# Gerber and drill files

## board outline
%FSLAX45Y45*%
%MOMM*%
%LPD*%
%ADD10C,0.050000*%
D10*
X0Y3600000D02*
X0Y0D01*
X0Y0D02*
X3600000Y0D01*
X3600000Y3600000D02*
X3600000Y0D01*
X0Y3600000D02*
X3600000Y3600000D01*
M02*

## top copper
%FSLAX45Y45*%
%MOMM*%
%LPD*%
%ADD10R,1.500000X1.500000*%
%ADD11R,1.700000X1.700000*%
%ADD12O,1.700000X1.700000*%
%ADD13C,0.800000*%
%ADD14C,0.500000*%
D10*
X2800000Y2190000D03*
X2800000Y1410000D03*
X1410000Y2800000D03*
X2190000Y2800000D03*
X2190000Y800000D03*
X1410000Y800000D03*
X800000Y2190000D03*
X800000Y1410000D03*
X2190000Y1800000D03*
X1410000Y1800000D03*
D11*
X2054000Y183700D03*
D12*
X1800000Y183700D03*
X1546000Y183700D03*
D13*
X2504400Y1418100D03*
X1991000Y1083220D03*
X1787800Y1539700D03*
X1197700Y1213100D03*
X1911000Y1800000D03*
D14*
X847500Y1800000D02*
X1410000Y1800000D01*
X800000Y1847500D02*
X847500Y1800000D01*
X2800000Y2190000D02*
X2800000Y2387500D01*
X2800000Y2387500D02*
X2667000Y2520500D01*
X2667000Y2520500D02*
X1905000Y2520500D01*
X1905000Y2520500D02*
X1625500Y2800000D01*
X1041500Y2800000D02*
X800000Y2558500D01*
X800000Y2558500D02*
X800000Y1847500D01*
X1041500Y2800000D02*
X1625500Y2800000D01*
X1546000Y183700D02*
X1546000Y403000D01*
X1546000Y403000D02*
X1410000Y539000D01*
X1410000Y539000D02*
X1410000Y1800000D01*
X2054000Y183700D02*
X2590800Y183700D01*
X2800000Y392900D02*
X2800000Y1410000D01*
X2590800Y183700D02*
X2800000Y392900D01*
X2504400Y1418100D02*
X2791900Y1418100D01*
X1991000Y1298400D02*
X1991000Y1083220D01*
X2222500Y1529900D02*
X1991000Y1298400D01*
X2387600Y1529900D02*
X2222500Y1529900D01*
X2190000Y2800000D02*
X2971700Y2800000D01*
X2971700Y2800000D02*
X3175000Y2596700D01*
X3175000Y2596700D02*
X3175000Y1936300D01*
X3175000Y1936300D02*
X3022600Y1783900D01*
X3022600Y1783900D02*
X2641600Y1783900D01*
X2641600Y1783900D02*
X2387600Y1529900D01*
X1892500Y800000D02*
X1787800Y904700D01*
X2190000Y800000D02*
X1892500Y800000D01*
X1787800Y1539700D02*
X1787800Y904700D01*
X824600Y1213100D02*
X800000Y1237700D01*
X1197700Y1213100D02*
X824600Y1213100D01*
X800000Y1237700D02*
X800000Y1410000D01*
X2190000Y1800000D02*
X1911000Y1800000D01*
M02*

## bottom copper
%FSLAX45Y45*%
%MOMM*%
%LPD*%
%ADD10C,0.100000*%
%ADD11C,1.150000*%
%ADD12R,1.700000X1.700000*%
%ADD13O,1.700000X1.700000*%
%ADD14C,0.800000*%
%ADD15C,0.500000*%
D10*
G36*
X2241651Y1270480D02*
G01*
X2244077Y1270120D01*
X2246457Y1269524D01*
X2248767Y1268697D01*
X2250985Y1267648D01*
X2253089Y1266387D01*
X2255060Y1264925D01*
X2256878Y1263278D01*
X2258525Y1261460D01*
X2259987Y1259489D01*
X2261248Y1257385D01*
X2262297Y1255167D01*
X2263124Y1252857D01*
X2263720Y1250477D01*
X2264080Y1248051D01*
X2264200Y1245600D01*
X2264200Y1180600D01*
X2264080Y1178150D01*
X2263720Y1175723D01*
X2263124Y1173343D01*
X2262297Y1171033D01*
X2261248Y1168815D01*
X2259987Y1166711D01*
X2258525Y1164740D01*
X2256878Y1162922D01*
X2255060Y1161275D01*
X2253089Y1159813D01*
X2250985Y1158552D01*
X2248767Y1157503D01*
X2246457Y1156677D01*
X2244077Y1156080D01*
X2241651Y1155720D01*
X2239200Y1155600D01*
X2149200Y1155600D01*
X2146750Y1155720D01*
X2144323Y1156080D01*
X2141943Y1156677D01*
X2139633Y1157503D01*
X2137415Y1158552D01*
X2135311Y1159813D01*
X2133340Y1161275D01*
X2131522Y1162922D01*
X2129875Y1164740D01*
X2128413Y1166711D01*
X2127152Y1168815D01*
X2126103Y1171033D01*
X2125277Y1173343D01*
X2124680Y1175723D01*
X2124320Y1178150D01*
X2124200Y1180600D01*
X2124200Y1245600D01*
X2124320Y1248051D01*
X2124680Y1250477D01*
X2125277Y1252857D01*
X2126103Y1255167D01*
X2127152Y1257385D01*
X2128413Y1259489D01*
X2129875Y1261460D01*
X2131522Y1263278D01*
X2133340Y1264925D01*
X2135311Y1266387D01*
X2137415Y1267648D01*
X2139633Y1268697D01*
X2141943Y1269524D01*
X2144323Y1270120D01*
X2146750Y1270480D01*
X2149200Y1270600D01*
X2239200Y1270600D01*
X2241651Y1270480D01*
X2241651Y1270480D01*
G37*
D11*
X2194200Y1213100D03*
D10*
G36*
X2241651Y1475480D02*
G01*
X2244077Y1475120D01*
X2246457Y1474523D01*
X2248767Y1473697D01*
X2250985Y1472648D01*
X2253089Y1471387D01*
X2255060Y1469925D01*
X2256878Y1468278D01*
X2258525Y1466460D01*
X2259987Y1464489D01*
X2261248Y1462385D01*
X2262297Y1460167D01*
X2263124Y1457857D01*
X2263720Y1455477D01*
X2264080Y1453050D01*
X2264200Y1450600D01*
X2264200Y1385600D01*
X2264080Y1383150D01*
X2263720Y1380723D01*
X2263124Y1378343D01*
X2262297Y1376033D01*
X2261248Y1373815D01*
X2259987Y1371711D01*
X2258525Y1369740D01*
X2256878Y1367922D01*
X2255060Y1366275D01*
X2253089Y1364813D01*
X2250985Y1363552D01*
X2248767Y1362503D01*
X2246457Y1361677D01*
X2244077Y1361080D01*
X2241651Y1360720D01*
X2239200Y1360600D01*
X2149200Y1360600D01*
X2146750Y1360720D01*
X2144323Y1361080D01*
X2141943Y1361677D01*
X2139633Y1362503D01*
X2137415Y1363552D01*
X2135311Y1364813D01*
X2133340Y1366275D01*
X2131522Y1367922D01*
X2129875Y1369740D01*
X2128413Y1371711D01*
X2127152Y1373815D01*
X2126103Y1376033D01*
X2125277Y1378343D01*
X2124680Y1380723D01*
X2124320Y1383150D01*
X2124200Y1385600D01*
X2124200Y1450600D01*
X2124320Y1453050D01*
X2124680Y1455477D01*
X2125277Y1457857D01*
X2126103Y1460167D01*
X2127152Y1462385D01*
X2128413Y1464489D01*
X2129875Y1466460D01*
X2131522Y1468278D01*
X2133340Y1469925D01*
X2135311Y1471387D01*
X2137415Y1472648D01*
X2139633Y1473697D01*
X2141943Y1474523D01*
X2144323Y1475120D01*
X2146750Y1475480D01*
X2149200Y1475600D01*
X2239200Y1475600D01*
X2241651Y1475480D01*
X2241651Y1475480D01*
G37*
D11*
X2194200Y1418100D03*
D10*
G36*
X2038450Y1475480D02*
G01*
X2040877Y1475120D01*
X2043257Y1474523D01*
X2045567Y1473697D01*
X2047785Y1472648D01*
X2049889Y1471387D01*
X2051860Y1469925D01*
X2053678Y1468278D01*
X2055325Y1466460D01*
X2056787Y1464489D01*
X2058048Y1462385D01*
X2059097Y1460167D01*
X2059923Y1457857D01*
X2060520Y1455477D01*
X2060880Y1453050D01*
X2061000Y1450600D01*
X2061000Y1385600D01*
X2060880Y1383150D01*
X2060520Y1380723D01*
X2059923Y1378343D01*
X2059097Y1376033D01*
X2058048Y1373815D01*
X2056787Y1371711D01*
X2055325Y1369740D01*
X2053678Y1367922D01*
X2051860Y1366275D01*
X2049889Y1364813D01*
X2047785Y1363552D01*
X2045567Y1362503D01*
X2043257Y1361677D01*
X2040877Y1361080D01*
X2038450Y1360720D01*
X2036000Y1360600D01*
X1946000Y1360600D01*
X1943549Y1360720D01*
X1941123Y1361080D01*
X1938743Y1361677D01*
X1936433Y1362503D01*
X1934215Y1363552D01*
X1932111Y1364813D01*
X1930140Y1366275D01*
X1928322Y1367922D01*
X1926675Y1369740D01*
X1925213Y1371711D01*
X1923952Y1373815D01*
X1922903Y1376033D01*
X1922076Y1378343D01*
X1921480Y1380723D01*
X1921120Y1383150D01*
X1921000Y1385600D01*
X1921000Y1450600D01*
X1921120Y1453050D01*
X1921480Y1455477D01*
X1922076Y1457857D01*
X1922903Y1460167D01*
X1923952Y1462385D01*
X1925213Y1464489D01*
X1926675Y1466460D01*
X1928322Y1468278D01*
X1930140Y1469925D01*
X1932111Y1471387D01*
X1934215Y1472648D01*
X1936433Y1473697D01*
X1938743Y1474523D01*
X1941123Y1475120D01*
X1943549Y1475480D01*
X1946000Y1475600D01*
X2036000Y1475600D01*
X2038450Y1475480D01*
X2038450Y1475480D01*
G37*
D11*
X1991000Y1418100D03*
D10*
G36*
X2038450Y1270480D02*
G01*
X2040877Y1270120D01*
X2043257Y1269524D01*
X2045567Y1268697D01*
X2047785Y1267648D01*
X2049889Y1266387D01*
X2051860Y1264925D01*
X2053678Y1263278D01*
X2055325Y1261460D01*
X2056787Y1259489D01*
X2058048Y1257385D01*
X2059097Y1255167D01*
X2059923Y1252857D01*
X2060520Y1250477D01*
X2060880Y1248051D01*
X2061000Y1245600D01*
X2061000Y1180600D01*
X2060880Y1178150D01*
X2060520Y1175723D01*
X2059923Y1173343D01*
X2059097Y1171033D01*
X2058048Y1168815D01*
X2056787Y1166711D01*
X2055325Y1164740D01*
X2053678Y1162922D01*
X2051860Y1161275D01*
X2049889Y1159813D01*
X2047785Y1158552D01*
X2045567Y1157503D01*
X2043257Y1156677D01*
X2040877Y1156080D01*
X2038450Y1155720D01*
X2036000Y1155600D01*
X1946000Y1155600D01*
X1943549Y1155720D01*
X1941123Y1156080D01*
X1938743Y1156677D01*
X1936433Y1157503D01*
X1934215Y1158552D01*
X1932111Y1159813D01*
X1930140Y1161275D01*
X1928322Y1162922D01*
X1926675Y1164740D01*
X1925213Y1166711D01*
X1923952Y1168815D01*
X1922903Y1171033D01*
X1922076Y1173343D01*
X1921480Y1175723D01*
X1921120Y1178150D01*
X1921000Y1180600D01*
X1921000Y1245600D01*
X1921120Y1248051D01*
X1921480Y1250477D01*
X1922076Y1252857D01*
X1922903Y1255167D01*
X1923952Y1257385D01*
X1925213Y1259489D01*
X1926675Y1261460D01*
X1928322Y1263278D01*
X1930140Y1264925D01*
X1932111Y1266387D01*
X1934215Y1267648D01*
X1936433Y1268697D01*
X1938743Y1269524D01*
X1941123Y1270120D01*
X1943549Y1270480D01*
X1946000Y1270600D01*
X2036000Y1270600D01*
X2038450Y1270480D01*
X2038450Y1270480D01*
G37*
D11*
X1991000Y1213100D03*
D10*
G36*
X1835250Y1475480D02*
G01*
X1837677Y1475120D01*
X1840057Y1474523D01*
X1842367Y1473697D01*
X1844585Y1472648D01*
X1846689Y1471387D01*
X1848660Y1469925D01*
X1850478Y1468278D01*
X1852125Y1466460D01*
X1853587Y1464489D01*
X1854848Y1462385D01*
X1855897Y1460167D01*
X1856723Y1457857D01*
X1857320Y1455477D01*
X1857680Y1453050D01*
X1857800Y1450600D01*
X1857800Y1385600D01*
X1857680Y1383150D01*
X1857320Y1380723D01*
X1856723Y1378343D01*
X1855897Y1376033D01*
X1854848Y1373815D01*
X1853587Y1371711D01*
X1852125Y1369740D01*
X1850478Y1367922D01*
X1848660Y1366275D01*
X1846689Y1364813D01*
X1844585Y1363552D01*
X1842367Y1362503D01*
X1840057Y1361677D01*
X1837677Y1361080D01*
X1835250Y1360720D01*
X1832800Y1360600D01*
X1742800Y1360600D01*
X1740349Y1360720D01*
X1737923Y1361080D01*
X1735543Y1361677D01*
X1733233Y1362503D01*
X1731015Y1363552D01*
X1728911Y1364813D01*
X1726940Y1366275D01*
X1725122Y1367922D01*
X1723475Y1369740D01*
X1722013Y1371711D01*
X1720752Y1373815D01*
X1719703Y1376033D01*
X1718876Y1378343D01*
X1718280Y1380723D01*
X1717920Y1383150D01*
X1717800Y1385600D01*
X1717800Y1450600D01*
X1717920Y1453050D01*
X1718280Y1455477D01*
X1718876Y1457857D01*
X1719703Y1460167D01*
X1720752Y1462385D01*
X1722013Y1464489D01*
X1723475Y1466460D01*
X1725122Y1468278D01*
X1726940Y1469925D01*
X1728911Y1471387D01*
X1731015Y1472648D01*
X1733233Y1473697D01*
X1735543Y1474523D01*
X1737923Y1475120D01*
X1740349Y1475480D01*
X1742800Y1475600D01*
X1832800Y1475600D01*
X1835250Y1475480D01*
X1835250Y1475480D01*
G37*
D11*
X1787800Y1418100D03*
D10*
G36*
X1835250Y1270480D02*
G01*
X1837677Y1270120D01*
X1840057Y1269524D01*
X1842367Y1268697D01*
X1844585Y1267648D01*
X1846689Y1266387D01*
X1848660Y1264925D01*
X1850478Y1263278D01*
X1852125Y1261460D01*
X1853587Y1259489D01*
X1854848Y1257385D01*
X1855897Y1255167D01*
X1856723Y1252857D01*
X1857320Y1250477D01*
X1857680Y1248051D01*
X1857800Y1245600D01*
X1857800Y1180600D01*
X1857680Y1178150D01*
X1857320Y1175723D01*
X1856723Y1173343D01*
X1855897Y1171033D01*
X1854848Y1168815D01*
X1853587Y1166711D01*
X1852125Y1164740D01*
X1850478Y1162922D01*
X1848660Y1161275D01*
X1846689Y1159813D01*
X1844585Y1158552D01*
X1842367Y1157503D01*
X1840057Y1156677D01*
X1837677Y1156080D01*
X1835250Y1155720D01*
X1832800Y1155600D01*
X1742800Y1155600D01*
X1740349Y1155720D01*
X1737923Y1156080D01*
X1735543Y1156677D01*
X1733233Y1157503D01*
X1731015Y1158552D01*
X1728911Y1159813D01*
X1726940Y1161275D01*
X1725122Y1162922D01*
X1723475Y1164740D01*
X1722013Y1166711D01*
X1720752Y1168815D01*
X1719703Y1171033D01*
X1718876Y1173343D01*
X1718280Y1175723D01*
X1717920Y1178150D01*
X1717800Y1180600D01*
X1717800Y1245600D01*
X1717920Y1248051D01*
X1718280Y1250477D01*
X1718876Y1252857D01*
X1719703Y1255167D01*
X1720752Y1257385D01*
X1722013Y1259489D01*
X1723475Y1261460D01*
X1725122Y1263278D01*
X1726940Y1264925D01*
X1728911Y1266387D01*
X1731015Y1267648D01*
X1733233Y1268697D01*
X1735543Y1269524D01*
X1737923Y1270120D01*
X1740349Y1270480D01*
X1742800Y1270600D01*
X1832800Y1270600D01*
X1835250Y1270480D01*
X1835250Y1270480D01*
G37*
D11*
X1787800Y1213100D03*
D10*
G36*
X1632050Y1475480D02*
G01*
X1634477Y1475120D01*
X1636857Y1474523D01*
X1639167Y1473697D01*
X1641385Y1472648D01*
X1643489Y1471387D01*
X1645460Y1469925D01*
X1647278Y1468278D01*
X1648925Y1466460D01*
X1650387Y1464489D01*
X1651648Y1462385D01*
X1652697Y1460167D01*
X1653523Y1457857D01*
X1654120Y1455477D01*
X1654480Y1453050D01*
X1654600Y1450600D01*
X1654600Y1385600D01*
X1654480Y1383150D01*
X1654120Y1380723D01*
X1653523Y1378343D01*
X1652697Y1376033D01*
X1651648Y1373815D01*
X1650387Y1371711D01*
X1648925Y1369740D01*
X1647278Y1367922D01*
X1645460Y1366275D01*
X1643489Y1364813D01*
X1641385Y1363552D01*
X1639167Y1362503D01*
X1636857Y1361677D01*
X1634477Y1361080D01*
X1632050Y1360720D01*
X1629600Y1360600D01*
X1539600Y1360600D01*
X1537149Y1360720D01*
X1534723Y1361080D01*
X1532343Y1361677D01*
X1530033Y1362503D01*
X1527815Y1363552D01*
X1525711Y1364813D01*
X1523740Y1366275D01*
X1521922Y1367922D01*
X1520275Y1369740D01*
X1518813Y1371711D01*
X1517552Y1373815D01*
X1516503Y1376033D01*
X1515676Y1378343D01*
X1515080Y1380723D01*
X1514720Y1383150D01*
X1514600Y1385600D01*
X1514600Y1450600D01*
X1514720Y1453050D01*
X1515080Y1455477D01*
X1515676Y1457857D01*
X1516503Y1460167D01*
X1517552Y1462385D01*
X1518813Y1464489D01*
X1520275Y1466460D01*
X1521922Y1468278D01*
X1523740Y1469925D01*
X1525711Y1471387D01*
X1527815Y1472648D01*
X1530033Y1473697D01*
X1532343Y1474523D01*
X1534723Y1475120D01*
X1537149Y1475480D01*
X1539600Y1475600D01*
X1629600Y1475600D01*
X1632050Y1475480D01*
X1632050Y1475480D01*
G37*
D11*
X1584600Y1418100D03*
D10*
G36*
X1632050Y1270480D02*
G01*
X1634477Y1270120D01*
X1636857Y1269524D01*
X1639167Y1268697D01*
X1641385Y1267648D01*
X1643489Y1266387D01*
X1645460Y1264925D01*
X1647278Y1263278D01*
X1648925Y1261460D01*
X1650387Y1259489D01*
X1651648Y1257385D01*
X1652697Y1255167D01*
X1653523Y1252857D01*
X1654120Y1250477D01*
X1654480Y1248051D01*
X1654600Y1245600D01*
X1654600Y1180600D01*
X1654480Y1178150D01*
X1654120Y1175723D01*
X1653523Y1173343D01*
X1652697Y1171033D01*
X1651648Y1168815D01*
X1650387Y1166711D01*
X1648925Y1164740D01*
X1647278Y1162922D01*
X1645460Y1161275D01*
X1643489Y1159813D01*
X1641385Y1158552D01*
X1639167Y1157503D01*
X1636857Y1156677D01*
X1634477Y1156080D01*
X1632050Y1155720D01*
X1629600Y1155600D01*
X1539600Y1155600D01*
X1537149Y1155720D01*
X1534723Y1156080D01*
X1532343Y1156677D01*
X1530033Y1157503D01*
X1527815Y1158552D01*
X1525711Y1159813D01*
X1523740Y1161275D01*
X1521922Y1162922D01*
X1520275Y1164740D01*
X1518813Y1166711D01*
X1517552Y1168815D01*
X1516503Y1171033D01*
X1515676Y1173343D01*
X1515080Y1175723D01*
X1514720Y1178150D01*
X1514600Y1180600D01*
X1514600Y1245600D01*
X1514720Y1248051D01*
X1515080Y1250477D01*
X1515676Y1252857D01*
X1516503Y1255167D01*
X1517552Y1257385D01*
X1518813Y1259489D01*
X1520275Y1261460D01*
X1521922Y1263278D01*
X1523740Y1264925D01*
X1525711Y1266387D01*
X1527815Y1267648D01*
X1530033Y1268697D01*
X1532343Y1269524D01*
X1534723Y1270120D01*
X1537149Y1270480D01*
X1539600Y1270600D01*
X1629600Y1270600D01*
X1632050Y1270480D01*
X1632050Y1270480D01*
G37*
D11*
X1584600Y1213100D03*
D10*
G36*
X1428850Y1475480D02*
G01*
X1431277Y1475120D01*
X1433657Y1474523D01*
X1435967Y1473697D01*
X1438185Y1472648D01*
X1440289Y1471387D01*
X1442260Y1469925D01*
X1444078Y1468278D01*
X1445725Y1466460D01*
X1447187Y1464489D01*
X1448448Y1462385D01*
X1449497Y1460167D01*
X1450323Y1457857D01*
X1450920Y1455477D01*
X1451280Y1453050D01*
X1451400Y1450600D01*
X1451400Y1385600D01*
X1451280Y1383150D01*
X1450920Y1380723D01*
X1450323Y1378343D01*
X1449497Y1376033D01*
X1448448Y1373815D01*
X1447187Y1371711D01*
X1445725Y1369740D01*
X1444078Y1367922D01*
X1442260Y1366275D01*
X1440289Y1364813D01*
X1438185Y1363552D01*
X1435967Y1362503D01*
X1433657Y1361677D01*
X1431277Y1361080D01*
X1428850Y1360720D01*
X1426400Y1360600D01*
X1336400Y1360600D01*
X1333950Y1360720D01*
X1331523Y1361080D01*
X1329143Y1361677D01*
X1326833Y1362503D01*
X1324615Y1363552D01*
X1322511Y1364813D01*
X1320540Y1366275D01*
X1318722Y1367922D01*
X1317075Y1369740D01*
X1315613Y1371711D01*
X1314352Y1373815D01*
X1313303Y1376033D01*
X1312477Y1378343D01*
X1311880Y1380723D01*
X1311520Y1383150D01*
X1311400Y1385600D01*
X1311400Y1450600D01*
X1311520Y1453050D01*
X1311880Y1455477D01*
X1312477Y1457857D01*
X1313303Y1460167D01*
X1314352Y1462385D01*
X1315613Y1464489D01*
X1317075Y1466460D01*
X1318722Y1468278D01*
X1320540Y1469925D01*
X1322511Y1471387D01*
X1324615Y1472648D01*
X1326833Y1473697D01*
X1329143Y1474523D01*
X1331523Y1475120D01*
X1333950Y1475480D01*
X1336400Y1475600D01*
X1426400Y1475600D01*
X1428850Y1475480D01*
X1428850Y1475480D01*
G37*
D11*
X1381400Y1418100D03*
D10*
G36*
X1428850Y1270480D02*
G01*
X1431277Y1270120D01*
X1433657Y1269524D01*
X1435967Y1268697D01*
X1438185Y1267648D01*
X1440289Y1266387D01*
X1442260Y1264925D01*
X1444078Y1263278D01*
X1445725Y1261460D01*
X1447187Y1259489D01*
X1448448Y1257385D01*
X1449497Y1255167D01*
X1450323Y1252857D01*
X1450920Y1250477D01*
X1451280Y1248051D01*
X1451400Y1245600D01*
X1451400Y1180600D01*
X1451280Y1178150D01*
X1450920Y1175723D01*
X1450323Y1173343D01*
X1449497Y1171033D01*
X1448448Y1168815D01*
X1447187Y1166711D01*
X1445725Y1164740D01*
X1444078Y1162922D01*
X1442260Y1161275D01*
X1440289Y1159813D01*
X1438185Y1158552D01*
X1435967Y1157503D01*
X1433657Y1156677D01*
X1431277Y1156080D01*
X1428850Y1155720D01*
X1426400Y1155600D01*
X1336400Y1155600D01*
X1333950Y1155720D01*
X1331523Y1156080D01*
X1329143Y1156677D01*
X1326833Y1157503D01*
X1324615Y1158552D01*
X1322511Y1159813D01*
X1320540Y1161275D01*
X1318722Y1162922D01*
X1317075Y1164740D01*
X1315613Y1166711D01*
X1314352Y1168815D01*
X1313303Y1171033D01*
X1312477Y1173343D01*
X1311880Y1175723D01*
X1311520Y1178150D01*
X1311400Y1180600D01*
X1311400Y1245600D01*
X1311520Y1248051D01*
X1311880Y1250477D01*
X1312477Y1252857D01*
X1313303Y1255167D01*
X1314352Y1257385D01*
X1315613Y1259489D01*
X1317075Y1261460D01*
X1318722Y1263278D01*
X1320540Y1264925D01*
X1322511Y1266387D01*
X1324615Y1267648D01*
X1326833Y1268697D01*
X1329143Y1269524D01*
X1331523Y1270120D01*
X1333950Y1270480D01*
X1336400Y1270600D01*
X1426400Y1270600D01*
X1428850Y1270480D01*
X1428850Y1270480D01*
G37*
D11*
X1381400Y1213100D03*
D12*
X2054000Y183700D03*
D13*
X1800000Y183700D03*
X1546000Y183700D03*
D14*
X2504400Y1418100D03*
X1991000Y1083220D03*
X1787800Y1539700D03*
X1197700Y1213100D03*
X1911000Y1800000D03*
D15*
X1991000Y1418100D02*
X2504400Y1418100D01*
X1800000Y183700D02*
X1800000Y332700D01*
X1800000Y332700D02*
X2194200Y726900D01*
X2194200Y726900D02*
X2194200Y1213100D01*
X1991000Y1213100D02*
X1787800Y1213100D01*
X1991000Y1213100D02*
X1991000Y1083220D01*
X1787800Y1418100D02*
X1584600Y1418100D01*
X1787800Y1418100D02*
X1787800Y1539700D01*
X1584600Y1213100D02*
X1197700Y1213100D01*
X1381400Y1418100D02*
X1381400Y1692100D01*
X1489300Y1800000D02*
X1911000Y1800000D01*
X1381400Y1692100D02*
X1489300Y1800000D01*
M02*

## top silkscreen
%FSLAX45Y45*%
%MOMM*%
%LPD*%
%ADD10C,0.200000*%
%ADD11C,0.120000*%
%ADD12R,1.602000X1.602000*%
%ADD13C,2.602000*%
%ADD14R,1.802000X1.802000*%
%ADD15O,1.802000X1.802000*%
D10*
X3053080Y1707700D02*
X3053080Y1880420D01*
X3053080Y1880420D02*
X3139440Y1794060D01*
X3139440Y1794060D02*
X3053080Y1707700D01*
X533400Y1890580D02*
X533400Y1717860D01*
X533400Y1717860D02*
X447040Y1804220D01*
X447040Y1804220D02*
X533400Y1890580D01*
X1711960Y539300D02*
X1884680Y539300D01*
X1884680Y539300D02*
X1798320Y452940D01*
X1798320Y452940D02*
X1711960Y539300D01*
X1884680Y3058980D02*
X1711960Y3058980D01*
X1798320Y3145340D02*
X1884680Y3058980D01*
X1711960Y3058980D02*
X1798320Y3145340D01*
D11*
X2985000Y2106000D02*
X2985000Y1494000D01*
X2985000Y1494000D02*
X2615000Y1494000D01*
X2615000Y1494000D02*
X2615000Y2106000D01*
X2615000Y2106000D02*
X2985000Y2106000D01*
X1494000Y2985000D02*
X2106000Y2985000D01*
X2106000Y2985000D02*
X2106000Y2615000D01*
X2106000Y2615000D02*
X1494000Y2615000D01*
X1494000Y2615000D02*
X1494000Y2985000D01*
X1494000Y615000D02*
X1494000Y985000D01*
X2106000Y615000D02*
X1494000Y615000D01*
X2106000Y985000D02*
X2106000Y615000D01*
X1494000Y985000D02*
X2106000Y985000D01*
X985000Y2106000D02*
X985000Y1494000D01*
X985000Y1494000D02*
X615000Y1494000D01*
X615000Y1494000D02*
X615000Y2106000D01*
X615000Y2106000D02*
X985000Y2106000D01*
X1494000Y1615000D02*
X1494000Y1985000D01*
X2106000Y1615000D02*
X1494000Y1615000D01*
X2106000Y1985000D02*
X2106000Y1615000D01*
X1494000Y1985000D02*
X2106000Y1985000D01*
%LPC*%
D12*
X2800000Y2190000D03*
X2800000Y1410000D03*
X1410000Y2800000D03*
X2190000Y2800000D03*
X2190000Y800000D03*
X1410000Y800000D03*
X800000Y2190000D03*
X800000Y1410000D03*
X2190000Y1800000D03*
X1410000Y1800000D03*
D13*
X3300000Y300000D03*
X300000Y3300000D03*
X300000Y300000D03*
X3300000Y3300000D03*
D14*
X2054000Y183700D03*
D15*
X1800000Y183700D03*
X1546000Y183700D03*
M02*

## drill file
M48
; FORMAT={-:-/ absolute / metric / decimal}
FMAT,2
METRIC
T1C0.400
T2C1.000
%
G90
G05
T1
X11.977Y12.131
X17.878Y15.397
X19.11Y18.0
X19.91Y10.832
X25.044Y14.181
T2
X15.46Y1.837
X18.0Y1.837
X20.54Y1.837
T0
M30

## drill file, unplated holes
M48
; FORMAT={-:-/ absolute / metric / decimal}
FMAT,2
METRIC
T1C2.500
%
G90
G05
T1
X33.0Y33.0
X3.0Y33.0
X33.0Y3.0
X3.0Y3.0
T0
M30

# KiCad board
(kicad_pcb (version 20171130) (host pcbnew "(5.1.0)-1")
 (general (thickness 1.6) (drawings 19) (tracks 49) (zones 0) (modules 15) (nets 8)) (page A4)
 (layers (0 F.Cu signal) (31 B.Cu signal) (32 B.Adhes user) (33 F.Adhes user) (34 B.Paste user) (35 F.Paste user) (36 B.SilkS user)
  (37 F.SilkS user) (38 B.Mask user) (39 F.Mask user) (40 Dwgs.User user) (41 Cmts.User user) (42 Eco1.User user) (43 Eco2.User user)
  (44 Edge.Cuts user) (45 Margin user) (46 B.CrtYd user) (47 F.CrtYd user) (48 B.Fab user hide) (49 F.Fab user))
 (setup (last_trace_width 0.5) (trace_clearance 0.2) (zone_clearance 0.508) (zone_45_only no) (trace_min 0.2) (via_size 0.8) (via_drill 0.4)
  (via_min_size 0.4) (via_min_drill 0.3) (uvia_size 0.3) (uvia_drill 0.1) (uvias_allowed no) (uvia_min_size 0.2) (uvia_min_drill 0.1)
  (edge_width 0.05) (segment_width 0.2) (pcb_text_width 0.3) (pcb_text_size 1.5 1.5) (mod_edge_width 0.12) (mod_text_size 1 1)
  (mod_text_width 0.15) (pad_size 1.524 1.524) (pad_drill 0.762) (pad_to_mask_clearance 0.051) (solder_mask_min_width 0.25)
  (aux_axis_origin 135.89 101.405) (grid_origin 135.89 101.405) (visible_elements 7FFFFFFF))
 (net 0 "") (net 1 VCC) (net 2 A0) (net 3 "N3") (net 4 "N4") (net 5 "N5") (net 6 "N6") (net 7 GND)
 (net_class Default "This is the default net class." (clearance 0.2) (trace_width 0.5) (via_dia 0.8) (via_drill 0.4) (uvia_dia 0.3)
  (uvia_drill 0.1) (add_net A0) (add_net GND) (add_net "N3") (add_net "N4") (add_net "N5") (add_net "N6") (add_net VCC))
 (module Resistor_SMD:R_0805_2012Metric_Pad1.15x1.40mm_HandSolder (layer B.Cu) (at 157.832 88.249 90)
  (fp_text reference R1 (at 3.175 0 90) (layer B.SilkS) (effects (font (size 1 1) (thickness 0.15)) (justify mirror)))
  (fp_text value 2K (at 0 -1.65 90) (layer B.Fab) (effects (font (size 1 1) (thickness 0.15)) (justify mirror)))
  (pad 1 smd roundrect (at -1.025 0 90) (size 1.15 1.4) (layers B.Cu B.Paste B.Mask) (roundrect_rratio 0.217391) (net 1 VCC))
  (pad 2 smd roundrect (at 1.025 0 90) (size 1.15 1.4) (layers B.Cu B.Paste B.Mask) (roundrect_rratio 0.217391) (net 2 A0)))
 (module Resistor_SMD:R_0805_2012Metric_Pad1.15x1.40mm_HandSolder (layer B.Cu) (at 155.8 88.249 270)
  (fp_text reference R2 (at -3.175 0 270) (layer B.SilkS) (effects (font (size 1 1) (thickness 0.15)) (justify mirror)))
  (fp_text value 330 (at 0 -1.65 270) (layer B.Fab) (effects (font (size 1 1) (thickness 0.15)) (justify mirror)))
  (pad 1 smd roundrect (at -1.025 0 270) (size 1.15 1.4) (layers B.Cu B.Paste B.Mask) (roundrect_rratio 0.217391) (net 2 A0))
  (pad 2 smd roundrect (at 1.025 0 270) (size 1.15 1.4) (layers B.Cu B.Paste B.Mask) (roundrect_rratio 0.217391) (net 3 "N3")))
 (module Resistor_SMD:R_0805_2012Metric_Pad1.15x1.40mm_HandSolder (layer B.Cu) (at 153.768 88.249 90)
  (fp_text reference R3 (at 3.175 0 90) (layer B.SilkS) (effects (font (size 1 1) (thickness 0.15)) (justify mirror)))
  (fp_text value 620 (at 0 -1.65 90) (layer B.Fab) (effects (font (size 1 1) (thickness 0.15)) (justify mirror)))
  (pad 2 smd roundrect (at 1.025 0 90) (size 1.15 1.4) (layers B.Cu B.Paste B.Mask) (roundrect_rratio 0.217391) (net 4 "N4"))
  (pad 1 smd roundrect (at -1.025 0 90) (size 1.15 1.4) (layers B.Cu B.Paste B.Mask) (roundrect_rratio 0.217391) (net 3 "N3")))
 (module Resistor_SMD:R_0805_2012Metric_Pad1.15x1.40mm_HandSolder (layer B.Cu) (at 151.736 88.249 270)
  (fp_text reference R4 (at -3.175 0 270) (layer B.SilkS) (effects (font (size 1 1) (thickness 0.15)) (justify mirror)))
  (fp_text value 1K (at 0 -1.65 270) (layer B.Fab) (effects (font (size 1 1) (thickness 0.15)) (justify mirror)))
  (pad 1 smd roundrect (at -1.025 0 270) (size 1.15 1.4) (layers B.Cu B.Paste B.Mask) (roundrect_rratio 0.217391) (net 4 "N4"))
  (pad 2 smd roundrect (at 1.025 0 270) (size 1.15 1.4) (layers B.Cu B.Paste B.Mask) (roundrect_rratio 0.217391) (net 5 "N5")))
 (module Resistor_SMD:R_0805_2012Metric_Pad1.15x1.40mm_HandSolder (layer B.Cu) (at 149.704 88.249 90)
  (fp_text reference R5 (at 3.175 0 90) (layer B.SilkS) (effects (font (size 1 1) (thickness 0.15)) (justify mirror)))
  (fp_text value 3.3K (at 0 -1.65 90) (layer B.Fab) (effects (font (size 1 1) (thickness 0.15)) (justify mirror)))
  (pad 2 smd roundrect (at 1.025 0 90) (size 1.15 1.4) (layers B.Cu B.Paste B.Mask) (roundrect_rratio 0.217391) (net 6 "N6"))
  (pad 1 smd roundrect (at -1.025 0 90) (size 1.15 1.4) (layers B.Cu B.Paste B.Mask) (roundrect_rratio 0.217391) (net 5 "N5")))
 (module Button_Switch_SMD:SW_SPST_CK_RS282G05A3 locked (layer F.Cu) (at 163.89 83.405 270)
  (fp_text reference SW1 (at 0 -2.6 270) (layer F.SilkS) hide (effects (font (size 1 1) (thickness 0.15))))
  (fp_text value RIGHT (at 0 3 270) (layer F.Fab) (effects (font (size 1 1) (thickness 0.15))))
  (fp_line (start -3.06 -1.85) (end 3.06 -1.85) (layer F.SilkS) (width 0.12))
  (fp_line (start 3.06 -1.85) (end 3.06 1.85) (layer F.SilkS) (width 0.12))
  (fp_line (start 3.06 1.85) (end -3.06 1.85) (layer F.SilkS) (width 0.12))
  (fp_line (start -3.06 1.85) (end -3.06 -1.85) (layer F.SilkS) (width 0.12))
  (pad 1 smd rect (at -3.9 0 270) (size 1.5 1.5) (layers F.Cu F.Paste F.Mask) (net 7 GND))
  (pad 2 smd rect (at 3.9 0 270) (size 1.5 1.5) (layers F.Cu F.Paste F.Mask) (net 2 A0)))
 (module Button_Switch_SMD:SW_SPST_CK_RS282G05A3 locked (layer F.Cu) (at 153.89 73.405)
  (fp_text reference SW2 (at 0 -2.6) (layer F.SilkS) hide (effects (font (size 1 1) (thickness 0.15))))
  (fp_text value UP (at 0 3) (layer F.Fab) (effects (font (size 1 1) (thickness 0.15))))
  (fp_line (start -3.06 -1.85) (end 3.06 -1.85) (layer F.SilkS) (width 0.12))
  (fp_line (start 3.06 -1.85) (end 3.06 1.85) (layer F.SilkS) (width 0.12))
  (fp_line (start 3.06 1.85) (end -3.06 1.85) (layer F.SilkS) (width 0.12))
  (fp_line (start -3.06 1.85) (end -3.06 -1.85) (layer F.SilkS) (width 0.12))
  (pad 1 smd rect (at -3.9 0) (size 1.5 1.5) (layers F.Cu F.Paste F.Mask) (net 7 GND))
  (pad 2 smd rect (at 3.9 0) (size 1.5 1.5) (layers F.Cu F.Paste F.Mask) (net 3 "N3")))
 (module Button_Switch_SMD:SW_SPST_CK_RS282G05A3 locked (layer F.Cu) (at 153.89 93.405)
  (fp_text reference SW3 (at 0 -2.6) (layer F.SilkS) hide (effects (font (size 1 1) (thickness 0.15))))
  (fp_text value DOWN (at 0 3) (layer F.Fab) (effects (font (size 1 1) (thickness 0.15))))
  (fp_line (start -3.06 1.85) (end -3.06 -1.85) (layer F.SilkS) (width 0.12))
  (fp_line (start 3.06 1.85) (end -3.06 1.85) (layer F.SilkS) (width 0.12))
  (fp_line (start 3.06 -1.85) (end 3.06 1.85) (layer F.SilkS) (width 0.12))
  (fp_line (start -3.06 -1.85) (end 3.06 -1.85) (layer F.SilkS) (width 0.12))
  (pad 2 smd rect (at 3.9 0) (size 1.5 1.5) (layers F.Cu F.Paste F.Mask) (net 4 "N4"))
  (pad 1 smd rect (at -3.9 0) (size 1.5 1.5) (layers F.Cu F.Paste F.Mask) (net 7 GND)))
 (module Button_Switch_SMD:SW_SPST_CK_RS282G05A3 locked (layer F.Cu) (at 143.89 83.405 270)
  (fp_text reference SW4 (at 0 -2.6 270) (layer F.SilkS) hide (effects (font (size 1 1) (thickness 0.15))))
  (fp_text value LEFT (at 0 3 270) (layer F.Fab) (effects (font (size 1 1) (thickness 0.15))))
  (fp_line (start -3.06 -1.85) (end 3.06 -1.85) (layer F.SilkS) (width 0.12))
  (fp_line (start 3.06 -1.85) (end 3.06 1.85) (layer F.SilkS) (width 0.12))
  (fp_line (start 3.06 1.85) (end -3.06 1.85) (layer F.SilkS) (width 0.12))
  (fp_line (start -3.06 1.85) (end -3.06 -1.85) (layer F.SilkS) (width 0.12))
  (pad 1 smd rect (at -3.9 0 270) (size 1.5 1.5) (layers F.Cu F.Paste F.Mask) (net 7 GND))
  (pad 2 smd rect (at 3.9 0 270) (size 1.5 1.5) (layers F.Cu F.Paste F.Mask) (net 5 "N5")))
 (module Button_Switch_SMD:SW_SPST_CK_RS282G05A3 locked (layer F.Cu) (at 153.89 83.405)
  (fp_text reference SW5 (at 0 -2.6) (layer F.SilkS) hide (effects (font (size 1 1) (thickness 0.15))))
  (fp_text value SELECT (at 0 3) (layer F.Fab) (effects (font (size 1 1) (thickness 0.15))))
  (fp_line (start -3.06 1.85) (end -3.06 -1.85) (layer F.SilkS) (width 0.12))
  (fp_line (start 3.06 1.85) (end -3.06 1.85) (layer F.SilkS) (width 0.12))
  (fp_line (start 3.06 -1.85) (end 3.06 1.85) (layer F.SilkS) (width 0.12))
  (fp_line (start -3.06 -1.85) (end 3.06 -1.85) (layer F.SilkS) (width 0.12))
  (pad 2 smd rect (at 3.9 0) (size 1.5 1.5) (layers F.Cu F.Paste F.Mask) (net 6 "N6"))
  (pad 1 smd rect (at -3.9 0) (size 1.5 1.5) (layers F.Cu F.Paste F.Mask) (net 7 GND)))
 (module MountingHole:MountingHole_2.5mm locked (layer F.Cu) (at 168.89 98.405)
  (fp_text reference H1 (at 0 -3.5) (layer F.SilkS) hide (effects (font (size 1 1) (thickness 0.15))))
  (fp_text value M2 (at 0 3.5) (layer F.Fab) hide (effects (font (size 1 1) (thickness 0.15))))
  (pad 1 np_thru_hole circle (at 0 0) (size 2.5 2.5) (drill 2.5) (layers *.Cu *.Mask)))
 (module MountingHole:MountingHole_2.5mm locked (layer F.Cu) (at 138.89 68.405)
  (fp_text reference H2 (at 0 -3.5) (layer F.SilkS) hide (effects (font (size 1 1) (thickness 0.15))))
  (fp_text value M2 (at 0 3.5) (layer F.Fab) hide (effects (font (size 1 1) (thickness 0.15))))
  (pad 1 np_thru_hole circle (at 0 0) (size 2.5 2.5) (drill 2.5) (layers *.Cu *.Mask)))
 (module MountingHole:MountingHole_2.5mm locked (layer F.Cu) (at 138.89 98.405)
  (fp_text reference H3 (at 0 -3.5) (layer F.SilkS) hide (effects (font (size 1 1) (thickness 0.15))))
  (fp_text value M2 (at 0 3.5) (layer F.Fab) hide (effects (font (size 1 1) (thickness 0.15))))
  (pad 1 np_thru_hole circle (at 0 0) (size 2.5 2.5) (drill 2.5) (layers *.Cu *.Mask)))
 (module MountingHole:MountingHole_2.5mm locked (layer F.Cu) (at 168.89 68.405)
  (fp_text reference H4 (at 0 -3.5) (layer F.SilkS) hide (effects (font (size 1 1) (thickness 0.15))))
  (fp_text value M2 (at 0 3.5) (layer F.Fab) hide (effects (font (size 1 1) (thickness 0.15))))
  (pad 1 np_thru_hole circle (at 0 0) (size 2.5 2.5) (drill 2.5) (layers *.Cu *.Mask)))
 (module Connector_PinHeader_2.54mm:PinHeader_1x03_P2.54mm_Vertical (layer B.Cu) (at 156.43 99.568 90)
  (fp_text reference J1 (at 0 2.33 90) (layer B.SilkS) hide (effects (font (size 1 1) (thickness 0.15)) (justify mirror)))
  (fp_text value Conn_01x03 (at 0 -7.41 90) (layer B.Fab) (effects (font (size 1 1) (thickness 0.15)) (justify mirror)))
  (pad 1 thru_hole rect (at 0 0 90) (size 1.7 1.7) (drill 1) (layers *.Cu *.Mask) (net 2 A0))
  (pad 2 thru_hole oval (at 0 -2.54 90) (size 1.7 1.7) (drill 1) (layers *.Cu *.Mask) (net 1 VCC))
  (pad 3 thru_hole oval (at 0 -5.08 90) (size 1.7 1.7) (drill 1) (layers *.Cu *.Mask) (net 7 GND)))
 (gr_line (start 166.4208 84.328) (end 166.4208 82.6008) (layer F.SilkS) (width 0.2))
 (gr_line (start 166.4208 82.6008) (end 167.2844 83.4644) (layer F.SilkS) (width 0.2))
 (gr_line (start 167.2844 83.4644) (end 166.4208 84.328) (layer F.SilkS) (width 0.2))
 (gr_line (start 141.224 82.4992) (end 141.224 84.2264) (layer F.SilkS) (width 0.2))
 (gr_line (start 141.224 84.2264) (end 140.3604 83.3628) (layer F.SilkS) (width 0.2))
 (gr_line (start 140.3604 83.3628) (end 141.224 82.4992) (layer F.SilkS) (width 0.2))
 (gr_line (start 153.0096 96.012) (end 154.7368 96.012) (layer F.SilkS) (width 0.2))
 (gr_line (start 154.7368 96.012) (end 153.8732 96.8756) (layer F.SilkS) (width 0.2))
 (gr_line (start 153.8732 96.8756) (end 153.0096 96.012) (layer F.SilkS) (width 0.2))
 (gr_line (start 154.7368 70.8152) (end 153.0096 70.8152) (layer F.SilkS) (width 0.2))
 (gr_line (start 153.8732 69.9516) (end 154.7368 70.8152) (layer F.SilkS) (width 0.2))
 (gr_line (start 153.0096 70.8152) (end 153.8732 69.9516) (layer F.SilkS) (width 0.2))
 (gr_line (start 135.89 65.405) (end 135.89 101.405) (layer Edge.Cuts) (width 0.05))
 (gr_line (start 135.89 101.405) (end 171.89 101.405) (layer Edge.Cuts) (width 0.05))
 (gr_line (start 171.89 65.405) (end 171.89 101.405) (layer Edge.Cuts) (width 0.05))
 (gr_line (start 135.89 65.405) (end 171.89 65.405) (layer Edge.Cuts) (width 0.05))
 (segment (start 144.365 83.405) (end 149.99 83.405) (width 0.5) (layer F.Cu) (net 7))
 (segment (start 143.89 82.93) (end 144.365 83.405) (width 0.5) (layer F.Cu) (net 7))
 (segment (start 163.89 79.505) (end 163.89 77.53) (width 0.5) (layer F.Cu) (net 7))
 (segment (start 163.89 77.53) (end 162.56 76.2) (width 0.5) (layer F.Cu) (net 7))
 (segment (start 162.56 76.2) (end 154.94 76.2) (width 0.5) (layer F.Cu) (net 7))
 (segment (start 154.94 76.2) (end 152.145 73.405) (width 0.5) (layer F.Cu) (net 7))
 (segment (start 146.305 73.405) (end 143.89 75.82) (width 0.5) (layer F.Cu) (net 7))
 (segment (start 143.89 75.82) (end 143.89 82.93) (width 0.5) (layer F.Cu) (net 7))
 (segment (start 146.305 73.405) (end 152.145 73.405) (width 0.5) (layer F.Cu) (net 7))
 (segment (start 151.35 99.568) (end 151.35 97.375) (width 0.5) (layer F.Cu) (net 7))
 (segment (start 151.35 97.375) (end 149.99 96.015) (width 0.5) (layer F.Cu) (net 7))
 (segment (start 149.99 96.015) (end 149.99 83.405) (width 0.5) (layer F.Cu) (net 7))
 (segment (start 156.43 99.568) (end 161.798 99.568) (width 0.5) (layer F.Cu) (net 2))
 (segment (start 163.89 97.476) (end 163.89 87.305) (width 0.5) (layer F.Cu) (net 2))
 (segment (start 161.798 99.568) (end 163.89 97.476) (width 0.5) (layer F.Cu) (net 2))
 (segment (start 160.934 87.224) (end 163.809 87.224) (width 0.5) (layer F.Cu) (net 2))
 (via (at 160.934 87.224) (size 0.8) (drill 0.4) (layers F.Cu B.Cu) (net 2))
 (segment (start 155.8 87.224) (end 160.934 87.224) (width 0.5) (layer B.Cu) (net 2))
 (segment (start 153.89 99.568) (end 153.89 98.078) (width 0.5) (layer B.Cu) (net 1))
 (segment (start 153.89 98.078) (end 157.832 94.136) (width 0.5) (layer B.Cu) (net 1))
 (segment (start 157.832 94.136) (end 157.832 89.274) (width 0.5) (layer B.Cu) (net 1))
 (segment (start 155.8 89.274) (end 153.768 89.274) (width 0.5) (layer B.Cu) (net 3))
 (segment (start 155.8 89.274) (end 155.8 90.5728) (width 0.5) (layer B.Cu) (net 3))
 (via (at 155.8 90.5728) (size 0.8) (drill 0.4) (layers F.Cu B.Cu) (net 3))
 (segment (start 155.8 88.421) (end 155.8 90.5728) (width 0.5) (layer F.Cu) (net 3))
 (segment (start 158.115 86.106) (end 155.8 88.421) (width 0.5) (layer F.Cu) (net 3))
 (segment (start 159.766 86.106) (end 158.115 86.106) (width 0.5) (layer F.Cu) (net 3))
 (segment (start 157.79 73.405) (end 165.607 73.405) (width 0.5) (layer F.Cu) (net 3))
 (segment (start 165.607 73.405) (end 167.64 75.438) (width 0.5) (layer F.Cu) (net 3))
 (segment (start 167.64 75.438) (end 167.64 82.042) (width 0.5) (layer F.Cu) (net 3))
 (segment (start 167.64 82.042) (end 166.116 83.566) (width 0.5) (layer F.Cu) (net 3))
 (segment (start 166.116 83.566) (end 162.306 83.566) (width 0.5) (layer F.Cu) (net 3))
 (segment (start 162.306 83.566) (end 159.766 86.106) (width 0.5) (layer F.Cu) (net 3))
 (segment (start 153.768 87.224) (end 151.736 87.224) (width 0.5) (layer B.Cu) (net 4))
 (segment (start 154.815 93.405) (end 153.768 92.358) (width 0.5) (layer F.Cu) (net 4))
 (segment (start 157.79 93.405) (end 154.815 93.405) (width 0.5) (layer F.Cu) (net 4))
 (segment (start 153.768 87.224) (end 153.768 86.008) (width 0.5) (layer B.Cu) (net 4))
 (via (at 153.768 86.008) (size 0.8) (drill 0.4) (layers F.Cu B.Cu) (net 4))
 (segment (start 153.768 86.008) (end 153.768 92.358) (width 0.5) (layer F.Cu) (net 4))
 (via (at 147.867 89.274) (size 0.8) (drill 0.4) (layers F.Cu B.Cu) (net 5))
 (segment (start 151.736 89.274) (end 147.867 89.274) (width 0.5) (layer B.Cu) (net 5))
 (segment (start 144.136 89.274) (end 143.89 89.028) (width 0.5) (layer F.Cu) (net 5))
 (segment (start 147.867 89.274) (end 144.136 89.274) (width 0.5) (layer F.Cu) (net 5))
 (segment (start 143.89 89.028) (end 143.89 87.305) (width 0.5) (layer F.Cu) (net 5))
 (via (at 155 83.405) (size 0.8) (drill 0.4) (layers F.Cu B.Cu) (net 6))
 (segment (start 149.704 87.224) (end 149.704 84.484) (width 0.5) (layer B.Cu) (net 6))
 (segment (start 150.783 83.405) (end 155 83.405) (width 0.5) (layer B.Cu) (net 6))
 (segment (start 149.704 84.484) (end 150.783 83.405) (width 0.5) (layer B.Cu) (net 6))
 (segment (start 157.79 83.405) (end 155 83.405) (width 0.5) (layer F.Cu) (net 6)))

